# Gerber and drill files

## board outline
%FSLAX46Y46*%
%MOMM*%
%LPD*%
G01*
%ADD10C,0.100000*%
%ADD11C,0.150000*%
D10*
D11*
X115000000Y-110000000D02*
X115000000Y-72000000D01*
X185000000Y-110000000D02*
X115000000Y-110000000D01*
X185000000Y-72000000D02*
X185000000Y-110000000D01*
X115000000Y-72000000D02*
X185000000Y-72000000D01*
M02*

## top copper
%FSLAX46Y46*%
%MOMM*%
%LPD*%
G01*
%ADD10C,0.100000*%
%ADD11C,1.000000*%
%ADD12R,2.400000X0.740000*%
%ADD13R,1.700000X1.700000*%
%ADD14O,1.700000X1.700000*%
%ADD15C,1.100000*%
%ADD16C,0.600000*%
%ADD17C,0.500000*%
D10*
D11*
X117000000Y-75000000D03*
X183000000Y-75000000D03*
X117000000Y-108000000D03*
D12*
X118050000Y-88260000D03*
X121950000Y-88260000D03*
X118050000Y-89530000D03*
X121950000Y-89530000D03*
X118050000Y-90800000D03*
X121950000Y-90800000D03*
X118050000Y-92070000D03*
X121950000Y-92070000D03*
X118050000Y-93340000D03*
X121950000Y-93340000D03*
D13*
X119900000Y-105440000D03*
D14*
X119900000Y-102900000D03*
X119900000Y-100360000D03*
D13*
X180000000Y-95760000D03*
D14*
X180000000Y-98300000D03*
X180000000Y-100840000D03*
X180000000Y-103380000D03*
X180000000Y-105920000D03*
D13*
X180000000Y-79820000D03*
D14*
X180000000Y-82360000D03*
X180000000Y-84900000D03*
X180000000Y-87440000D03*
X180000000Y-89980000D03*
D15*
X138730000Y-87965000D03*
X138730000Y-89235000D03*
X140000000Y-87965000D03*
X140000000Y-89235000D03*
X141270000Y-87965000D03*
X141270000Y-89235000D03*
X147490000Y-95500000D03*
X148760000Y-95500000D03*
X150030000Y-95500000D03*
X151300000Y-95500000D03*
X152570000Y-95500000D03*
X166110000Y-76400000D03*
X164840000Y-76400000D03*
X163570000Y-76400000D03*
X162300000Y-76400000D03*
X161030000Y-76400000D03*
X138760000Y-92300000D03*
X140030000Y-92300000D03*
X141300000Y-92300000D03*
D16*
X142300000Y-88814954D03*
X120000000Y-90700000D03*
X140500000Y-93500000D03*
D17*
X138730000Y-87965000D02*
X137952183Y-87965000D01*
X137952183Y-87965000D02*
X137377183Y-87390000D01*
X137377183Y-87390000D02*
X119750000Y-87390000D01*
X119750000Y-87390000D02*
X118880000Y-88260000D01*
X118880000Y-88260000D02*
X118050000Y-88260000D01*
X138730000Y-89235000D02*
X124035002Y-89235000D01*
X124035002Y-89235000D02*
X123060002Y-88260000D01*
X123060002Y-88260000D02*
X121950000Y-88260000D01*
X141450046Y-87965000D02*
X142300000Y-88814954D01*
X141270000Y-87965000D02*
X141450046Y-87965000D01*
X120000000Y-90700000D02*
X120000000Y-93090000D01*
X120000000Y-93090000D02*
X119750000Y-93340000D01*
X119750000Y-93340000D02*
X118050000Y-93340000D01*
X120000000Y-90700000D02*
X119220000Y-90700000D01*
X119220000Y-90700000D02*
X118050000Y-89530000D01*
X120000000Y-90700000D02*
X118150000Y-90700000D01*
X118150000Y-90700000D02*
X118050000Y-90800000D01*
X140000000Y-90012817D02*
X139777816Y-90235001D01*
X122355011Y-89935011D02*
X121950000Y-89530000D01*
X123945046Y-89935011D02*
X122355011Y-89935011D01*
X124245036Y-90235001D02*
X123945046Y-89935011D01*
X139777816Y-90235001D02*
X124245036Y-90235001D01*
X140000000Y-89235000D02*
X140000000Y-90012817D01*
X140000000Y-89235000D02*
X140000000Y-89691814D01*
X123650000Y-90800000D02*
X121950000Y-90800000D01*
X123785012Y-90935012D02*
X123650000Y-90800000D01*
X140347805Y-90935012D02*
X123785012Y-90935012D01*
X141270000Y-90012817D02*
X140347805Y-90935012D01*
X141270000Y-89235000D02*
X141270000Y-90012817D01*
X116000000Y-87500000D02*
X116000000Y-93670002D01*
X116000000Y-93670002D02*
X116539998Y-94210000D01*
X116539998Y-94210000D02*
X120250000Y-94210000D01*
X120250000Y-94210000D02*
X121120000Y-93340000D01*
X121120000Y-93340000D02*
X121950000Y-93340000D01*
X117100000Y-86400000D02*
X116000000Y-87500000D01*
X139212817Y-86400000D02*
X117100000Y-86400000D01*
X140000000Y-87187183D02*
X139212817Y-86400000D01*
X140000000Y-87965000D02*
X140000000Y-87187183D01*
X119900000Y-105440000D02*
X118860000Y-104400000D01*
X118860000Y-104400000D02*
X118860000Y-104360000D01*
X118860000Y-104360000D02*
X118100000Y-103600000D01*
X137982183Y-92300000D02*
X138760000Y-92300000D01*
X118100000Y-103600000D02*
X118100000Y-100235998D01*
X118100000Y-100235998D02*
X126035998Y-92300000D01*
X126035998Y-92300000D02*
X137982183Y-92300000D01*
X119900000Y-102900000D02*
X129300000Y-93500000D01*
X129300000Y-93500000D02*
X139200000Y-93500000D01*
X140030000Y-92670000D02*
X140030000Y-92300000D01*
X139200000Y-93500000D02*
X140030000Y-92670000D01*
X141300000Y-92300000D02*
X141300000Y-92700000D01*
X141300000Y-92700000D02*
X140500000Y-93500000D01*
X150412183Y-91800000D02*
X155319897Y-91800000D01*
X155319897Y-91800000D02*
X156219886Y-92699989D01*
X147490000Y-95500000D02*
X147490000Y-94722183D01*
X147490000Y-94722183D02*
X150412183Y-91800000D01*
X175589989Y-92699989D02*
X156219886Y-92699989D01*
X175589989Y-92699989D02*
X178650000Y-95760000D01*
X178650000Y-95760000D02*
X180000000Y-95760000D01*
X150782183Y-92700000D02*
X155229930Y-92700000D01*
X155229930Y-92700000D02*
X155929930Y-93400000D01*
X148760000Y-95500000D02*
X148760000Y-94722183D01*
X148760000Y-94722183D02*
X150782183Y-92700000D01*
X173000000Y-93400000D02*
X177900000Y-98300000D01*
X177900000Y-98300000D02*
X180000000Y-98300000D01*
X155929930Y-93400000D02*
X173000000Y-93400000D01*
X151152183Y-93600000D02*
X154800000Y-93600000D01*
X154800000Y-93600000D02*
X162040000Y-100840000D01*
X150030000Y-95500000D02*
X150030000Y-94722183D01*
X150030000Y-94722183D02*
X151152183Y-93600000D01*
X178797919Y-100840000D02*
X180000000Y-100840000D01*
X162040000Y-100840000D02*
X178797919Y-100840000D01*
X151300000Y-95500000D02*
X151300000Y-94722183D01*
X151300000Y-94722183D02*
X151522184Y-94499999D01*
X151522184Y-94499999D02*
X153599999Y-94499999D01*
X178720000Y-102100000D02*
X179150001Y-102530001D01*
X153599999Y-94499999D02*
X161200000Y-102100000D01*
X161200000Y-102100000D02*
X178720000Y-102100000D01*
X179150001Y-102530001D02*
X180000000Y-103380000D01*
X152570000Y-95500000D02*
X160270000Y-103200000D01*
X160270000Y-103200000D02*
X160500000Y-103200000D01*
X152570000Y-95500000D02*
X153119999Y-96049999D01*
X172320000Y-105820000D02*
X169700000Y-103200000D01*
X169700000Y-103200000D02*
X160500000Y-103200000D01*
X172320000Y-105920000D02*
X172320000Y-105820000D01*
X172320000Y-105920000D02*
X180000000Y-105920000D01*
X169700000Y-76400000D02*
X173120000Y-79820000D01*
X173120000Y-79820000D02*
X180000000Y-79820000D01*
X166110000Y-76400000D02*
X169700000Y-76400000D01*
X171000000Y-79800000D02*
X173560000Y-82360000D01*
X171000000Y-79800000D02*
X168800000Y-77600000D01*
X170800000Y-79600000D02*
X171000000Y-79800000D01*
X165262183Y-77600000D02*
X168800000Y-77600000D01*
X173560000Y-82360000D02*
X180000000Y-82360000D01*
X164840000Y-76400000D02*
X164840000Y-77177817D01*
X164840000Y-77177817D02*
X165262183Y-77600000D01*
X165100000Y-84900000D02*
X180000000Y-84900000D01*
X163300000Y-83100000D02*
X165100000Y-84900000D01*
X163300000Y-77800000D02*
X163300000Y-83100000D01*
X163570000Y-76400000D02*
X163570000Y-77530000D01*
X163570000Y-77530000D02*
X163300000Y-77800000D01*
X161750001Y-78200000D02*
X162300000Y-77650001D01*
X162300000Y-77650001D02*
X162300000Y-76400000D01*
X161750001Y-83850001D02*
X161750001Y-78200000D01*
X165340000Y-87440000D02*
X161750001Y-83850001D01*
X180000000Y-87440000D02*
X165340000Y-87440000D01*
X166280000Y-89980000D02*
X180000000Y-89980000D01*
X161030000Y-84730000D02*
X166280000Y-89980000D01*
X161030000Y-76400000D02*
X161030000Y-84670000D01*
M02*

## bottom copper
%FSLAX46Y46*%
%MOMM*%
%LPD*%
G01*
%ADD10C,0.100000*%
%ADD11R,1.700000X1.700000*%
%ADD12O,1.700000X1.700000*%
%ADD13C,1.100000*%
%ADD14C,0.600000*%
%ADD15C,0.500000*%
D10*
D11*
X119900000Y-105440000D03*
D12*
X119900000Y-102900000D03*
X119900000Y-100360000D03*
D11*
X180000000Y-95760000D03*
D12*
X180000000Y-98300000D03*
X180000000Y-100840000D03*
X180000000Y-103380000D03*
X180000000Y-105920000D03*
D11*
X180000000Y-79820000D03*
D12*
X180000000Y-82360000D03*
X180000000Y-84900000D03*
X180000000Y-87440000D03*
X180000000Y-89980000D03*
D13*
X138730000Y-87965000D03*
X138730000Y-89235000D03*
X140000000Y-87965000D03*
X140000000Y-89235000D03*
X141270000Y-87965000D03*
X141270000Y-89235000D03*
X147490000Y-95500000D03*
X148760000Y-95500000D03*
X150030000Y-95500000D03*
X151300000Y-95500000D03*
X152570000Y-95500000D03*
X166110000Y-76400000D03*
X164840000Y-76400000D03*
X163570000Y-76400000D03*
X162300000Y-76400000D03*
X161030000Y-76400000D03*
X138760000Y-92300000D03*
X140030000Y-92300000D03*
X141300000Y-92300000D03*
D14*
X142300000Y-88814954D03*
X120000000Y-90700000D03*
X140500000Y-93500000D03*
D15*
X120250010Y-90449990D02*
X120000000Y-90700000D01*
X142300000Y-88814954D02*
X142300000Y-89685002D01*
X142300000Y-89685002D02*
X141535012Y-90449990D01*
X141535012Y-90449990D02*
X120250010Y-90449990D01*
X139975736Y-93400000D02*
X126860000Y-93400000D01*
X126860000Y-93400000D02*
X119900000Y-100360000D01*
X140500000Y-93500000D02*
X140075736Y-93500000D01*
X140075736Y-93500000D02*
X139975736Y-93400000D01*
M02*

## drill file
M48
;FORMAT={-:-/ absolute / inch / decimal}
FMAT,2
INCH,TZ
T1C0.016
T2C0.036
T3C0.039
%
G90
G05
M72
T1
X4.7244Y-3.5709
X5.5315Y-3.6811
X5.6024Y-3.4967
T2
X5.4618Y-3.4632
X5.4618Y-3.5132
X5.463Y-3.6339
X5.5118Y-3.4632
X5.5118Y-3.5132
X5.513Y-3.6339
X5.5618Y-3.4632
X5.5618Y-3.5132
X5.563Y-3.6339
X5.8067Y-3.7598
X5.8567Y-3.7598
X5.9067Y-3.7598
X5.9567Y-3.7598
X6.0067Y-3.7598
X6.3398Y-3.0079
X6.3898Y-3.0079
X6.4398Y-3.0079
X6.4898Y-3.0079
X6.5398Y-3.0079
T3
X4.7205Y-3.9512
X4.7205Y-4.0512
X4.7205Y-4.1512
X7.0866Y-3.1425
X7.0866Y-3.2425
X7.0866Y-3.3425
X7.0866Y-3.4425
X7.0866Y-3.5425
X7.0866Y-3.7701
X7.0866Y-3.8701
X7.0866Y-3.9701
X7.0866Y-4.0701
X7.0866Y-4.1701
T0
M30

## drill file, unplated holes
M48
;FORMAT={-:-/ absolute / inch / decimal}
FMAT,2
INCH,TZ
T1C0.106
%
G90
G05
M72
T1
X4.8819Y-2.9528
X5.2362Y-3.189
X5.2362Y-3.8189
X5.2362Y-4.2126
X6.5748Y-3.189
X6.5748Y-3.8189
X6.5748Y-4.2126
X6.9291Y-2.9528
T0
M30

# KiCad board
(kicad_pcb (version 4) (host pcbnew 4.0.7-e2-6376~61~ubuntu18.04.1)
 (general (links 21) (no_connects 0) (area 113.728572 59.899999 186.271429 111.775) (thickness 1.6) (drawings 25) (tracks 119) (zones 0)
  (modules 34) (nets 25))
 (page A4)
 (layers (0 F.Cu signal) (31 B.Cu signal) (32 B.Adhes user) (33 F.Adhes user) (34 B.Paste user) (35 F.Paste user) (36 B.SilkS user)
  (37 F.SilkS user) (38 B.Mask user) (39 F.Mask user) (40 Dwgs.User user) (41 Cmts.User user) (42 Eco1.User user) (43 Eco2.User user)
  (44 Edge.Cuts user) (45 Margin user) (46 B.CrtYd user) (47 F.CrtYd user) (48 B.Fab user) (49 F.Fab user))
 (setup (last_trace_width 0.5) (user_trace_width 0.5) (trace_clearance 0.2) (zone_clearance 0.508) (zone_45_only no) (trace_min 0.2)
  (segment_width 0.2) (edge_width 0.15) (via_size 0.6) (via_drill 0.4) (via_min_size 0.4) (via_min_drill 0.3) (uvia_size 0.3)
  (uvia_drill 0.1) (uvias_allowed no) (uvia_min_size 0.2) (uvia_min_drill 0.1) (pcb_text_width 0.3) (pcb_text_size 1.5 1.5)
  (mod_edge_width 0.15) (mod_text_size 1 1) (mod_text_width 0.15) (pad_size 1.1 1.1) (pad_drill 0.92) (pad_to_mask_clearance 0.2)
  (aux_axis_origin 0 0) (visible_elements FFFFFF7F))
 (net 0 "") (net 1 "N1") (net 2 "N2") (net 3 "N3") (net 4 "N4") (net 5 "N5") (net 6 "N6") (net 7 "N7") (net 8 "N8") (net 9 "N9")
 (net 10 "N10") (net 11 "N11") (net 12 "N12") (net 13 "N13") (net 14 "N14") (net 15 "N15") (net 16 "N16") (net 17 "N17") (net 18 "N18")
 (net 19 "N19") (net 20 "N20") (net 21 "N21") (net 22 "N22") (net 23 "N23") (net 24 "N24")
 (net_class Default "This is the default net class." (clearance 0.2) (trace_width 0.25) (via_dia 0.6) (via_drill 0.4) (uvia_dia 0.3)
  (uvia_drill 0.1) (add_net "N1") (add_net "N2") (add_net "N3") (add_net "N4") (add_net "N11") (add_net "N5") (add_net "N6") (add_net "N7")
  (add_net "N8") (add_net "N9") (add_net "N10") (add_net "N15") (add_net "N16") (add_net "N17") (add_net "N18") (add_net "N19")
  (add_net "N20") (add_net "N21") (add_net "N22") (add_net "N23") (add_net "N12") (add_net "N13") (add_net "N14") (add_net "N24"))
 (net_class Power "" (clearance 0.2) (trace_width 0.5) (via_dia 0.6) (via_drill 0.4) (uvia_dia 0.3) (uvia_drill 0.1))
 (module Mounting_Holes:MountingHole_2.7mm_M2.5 (layer F.Cu) (at 176 75)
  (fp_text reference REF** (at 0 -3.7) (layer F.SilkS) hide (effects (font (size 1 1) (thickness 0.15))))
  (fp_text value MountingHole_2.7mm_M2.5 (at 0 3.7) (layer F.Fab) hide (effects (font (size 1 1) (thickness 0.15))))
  (pad 1 np_thru_hole circle (at 0 0) (size 2.7 2.7) (drill 2.7) (layers *.Cu *.Mask)))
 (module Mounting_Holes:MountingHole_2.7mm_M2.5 (layer F.Cu) (at 124 75)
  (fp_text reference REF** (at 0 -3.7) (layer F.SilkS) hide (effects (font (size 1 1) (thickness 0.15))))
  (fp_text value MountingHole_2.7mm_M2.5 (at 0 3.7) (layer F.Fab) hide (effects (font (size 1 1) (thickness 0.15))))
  (pad 1 np_thru_hole circle (at 0 0) (size 2.7 2.7) (drill 2.7) (layers *.Cu *.Mask)))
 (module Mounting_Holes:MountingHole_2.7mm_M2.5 (layer F.Cu) (at 167 107)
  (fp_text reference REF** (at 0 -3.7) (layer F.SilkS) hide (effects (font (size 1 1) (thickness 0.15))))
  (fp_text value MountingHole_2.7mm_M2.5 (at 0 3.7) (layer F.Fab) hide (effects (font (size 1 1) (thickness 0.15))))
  (pad 1 np_thru_hole circle (at 0 0) (size 2.7 2.7) (drill 2.7) (layers *.Cu *.Mask)))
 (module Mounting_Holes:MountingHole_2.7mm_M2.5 (layer F.Cu) (at 133 107)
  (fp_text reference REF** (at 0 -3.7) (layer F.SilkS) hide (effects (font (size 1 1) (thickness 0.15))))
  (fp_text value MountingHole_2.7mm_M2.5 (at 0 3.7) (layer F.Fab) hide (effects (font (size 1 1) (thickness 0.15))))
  (pad 1 np_thru_hole circle (at 0 0) (size 2.7 2.7) (drill 2.7) (layers *.Cu *.Mask)))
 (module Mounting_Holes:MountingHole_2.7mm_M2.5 (layer F.Cu) (at 167 81)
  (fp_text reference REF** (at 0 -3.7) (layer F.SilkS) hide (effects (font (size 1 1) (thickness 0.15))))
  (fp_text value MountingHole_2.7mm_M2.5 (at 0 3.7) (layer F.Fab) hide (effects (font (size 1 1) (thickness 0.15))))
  (pad 1 np_thru_hole circle (at 0 0) (size 2.7 2.7) (drill 2.7) (layers *.Cu *.Mask)))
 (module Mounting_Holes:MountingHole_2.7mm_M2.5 (layer F.Cu) (at 133 97)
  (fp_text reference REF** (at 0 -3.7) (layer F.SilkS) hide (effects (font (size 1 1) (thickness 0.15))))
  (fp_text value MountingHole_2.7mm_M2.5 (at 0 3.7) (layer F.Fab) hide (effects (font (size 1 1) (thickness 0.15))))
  (pad 1 np_thru_hole circle (at 0 0) (size 2.7 2.7) (drill 2.7) (layers *.Cu *.Mask)))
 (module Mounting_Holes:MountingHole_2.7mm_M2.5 (layer F.Cu) (at 167 97)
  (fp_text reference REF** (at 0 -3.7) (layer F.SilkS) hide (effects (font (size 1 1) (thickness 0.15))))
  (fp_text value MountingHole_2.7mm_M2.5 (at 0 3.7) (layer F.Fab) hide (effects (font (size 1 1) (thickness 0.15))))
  (pad 1 np_thru_hole circle (at 0 0) (size 2.7 2.7) (drill 2.7) (layers *.Cu *.Mask)))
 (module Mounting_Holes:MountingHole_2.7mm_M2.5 (layer F.Cu) (at 133 81)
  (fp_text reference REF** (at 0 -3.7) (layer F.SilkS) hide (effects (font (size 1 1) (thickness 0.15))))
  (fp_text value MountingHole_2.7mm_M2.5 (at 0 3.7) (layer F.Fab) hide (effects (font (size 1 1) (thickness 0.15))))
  (pad 1 np_thru_hole circle (at 0 0) (size 2.7 2.7) (drill 2.7) (layers *.Cu *.Mask)))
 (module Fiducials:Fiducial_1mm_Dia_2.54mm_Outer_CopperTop (layer F.Cu) (at 117 75)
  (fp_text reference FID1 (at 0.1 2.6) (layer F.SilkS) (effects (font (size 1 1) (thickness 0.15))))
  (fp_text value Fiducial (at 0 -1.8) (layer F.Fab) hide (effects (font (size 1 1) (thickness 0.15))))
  (pad ~ smd circle (at 0 0) (size 1 1) (layers F.Cu F.Mask) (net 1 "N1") (solder_mask_margin 0.77) (clearance 0.77)))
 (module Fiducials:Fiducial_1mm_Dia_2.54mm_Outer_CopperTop (layer F.Cu) (at 183 75)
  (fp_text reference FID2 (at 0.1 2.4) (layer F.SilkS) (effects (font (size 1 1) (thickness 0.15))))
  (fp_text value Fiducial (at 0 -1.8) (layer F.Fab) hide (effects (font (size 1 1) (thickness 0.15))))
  (pad ~ smd circle (at 0 0) (size 1 1) (layers F.Cu F.Mask) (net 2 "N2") (solder_mask_margin 0.77) (clearance 0.77)))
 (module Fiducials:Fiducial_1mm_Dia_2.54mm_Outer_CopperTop (layer F.Cu) (at 117 108)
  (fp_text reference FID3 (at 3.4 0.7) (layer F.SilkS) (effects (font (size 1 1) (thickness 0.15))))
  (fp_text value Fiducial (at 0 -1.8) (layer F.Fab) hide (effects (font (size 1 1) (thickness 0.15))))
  (pad ~ smd circle (at 0 0) (size 1 1) (layers F.Cu F.Mask) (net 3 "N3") (solder_mask_margin 0.77) (clearance 0.77)))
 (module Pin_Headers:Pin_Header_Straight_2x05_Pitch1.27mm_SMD (layer F.Cu) (at 120 90.8)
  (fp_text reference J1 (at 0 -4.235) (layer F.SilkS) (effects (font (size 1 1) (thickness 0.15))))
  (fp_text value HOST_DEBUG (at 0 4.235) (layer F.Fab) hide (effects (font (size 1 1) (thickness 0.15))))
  (pad 1 smd rect (at -1.95 -2.54) (size 2.4 0.74) (layers F.Cu F.Paste F.Mask) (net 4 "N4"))
  (pad 2 smd rect (at 1.95 -2.54) (size 2.4 0.74) (layers F.Cu F.Paste F.Mask) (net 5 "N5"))
  (pad 3 smd rect (at -1.95 -1.27) (size 2.4 0.74) (layers F.Cu F.Paste F.Mask) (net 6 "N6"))
  (pad 4 smd rect (at 1.95 -1.27) (size 2.4 0.74) (layers F.Cu F.Paste F.Mask) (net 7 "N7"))
  (pad 5 smd rect (at -1.95 0) (size 2.4 0.74) (layers F.Cu F.Paste F.Mask) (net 6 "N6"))
  (pad 6 smd rect (at 1.95 0) (size 2.4 0.74) (layers F.Cu F.Paste F.Mask) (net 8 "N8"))
  (pad 7 smd rect (at -1.95 1.27) (size 2.4 0.74) (layers F.Cu F.Paste F.Mask) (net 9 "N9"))
  (pad 8 smd rect (at 1.95 1.27) (size 2.4 0.74) (layers F.Cu F.Paste F.Mask) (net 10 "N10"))
  (pad 9 smd rect (at -1.95 2.54) (size 2.4 0.74) (layers F.Cu F.Paste F.Mask) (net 6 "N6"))
  (pad 10 smd rect (at 1.95 2.54) (size 2.4 0.74) (layers F.Cu F.Paste F.Mask) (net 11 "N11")))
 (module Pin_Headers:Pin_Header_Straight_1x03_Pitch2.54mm (layer F.Cu) (at 119.9 105.44 180)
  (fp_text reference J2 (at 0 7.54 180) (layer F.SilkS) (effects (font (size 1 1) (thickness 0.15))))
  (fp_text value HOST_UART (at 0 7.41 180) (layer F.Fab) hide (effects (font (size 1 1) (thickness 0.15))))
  (pad 1 thru_hole rect (at 0 0 180) (size 1.7 1.7) (drill 1) (layers *.Cu *.Mask) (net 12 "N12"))
  (pad 2 thru_hole oval (at 0 2.54 180) (size 1.7 1.7) (drill 1) (layers *.Cu *.Mask) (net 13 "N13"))
  (pad 3 thru_hole oval (at 0 5.08 180) (size 1.7 1.7) (drill 1) (layers *.Cu *.Mask) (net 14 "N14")))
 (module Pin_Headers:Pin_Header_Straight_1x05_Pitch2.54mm (layer F.Cu) (at 180 95.76)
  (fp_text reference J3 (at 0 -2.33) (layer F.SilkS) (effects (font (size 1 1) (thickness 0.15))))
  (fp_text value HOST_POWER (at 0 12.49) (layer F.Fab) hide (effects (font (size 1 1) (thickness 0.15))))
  (pad 1 thru_hole rect (at 0 0) (size 1.7 1.7) (drill 1) (layers *.Cu *.Mask) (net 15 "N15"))
  (pad 2 thru_hole oval (at 0 2.54) (size 1.7 1.7) (drill 1) (layers *.Cu *.Mask) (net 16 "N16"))
  (pad 3 thru_hole oval (at 0 5.08) (size 1.7 1.7) (drill 1) (layers *.Cu *.Mask) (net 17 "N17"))
  (pad 4 thru_hole oval (at 0 7.62) (size 1.7 1.7) (drill 1) (layers *.Cu *.Mask) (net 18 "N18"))
  (pad 5 thru_hole oval (at 0 10.16) (size 1.7 1.7) (drill 1) (layers *.Cu *.Mask) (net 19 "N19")))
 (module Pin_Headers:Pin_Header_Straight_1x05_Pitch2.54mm (layer F.Cu) (at 180 79.82)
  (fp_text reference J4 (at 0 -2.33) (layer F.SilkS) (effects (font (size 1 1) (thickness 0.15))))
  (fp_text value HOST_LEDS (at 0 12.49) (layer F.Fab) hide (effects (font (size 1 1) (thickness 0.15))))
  (pad 1 thru_hole rect (at 0 0) (size 1.7 1.7) (drill 1) (layers *.Cu *.Mask) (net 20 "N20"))
  (pad 2 thru_hole oval (at 0 2.54) (size 1.7 1.7) (drill 1) (layers *.Cu *.Mask) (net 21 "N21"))
  (pad 3 thru_hole oval (at 0 5.08) (size 1.7 1.7) (drill 1) (layers *.Cu *.Mask) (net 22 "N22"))
  (pad 4 thru_hole oval (at 0 7.62) (size 1.7 1.7) (drill 1) (layers *.Cu *.Mask) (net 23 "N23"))
  (pad 5 thru_hole oval (at 0 10.16) (size 1.7 1.7) (drill 1) (layers *.Cu *.Mask) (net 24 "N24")))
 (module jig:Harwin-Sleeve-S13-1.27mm (layer F.Cu) (at 138.73 87.965)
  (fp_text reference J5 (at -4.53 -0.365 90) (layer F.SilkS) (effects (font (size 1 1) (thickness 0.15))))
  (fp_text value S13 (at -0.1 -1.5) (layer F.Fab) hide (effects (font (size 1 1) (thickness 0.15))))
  (pad 1 thru_hole circle (at 0 0) (size 1.1 1.1) (drill 0.92) (layers *.Cu *.Mask) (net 4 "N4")))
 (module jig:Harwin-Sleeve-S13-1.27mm (layer F.Cu) (at 138.73 89.235)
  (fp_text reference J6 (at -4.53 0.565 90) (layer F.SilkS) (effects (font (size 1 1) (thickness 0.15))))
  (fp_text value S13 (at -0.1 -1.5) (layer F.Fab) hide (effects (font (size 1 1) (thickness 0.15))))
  (pad 1 thru_hole circle (at 0 0) (size 1.1 1.1) (drill 0.92) (layers *.Cu *.Mask) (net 5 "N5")))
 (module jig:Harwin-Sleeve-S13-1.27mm (layer F.Cu) (at 140 87.965)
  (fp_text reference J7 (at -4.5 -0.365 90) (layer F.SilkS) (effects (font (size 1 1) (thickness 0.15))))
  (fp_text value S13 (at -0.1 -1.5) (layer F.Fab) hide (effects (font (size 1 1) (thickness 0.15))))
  (pad 1 thru_hole circle (at 0 0) (size 1.1 1.1) (drill 0.92) (layers *.Cu *.Mask) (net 11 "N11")))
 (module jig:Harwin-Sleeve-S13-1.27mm (layer F.Cu) (at 140 89.235)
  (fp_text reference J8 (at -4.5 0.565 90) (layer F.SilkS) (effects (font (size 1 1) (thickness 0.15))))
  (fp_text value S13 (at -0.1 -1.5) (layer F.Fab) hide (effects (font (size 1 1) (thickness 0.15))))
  (pad 1 thru_hole circle (at 0 0) (size 1.1 1.1) (drill 0.92) (layers *.Cu *.Mask) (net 7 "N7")))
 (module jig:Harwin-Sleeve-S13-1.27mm (layer F.Cu) (at 141.27 87.965)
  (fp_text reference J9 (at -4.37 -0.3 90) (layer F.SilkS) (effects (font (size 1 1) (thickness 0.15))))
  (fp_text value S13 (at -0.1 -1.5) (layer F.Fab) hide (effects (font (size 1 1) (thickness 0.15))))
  (pad 1 thru_hole circle (at 0 0) (size 1.1 1.1) (drill 0.92) (layers *.Cu *.Mask) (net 6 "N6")))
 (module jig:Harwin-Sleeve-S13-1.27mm (layer F.Cu) (at 141.27 89.235)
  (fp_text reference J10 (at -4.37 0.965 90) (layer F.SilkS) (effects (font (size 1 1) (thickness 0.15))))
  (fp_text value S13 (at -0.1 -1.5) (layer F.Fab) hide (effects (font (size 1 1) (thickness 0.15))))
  (pad 1 thru_hole circle (at 0 0) (size 1.1 1.1) (drill 0.92) (layers *.Cu *.Mask) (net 8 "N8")))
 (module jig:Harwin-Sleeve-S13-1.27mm (layer F.Cu) (at 147.49 93.5)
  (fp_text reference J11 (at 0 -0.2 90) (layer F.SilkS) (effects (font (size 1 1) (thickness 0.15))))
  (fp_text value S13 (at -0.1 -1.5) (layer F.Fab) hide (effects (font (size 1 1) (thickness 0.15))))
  (pad 1 thru_hole circle (at 0 2) (size 1.1 1.1) (drill 0.92) (layers *.Cu *.Mask) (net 15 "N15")))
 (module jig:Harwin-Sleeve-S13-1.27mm (layer F.Cu) (at 148.76 93.5)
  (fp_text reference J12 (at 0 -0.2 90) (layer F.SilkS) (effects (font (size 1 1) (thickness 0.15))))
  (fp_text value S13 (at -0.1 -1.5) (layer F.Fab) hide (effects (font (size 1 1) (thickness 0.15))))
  (pad 1 thru_hole circle (at 0 2) (size 1.1 1.1) (drill 0.92) (layers *.Cu *.Mask) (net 16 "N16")))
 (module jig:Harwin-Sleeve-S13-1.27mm (layer F.Cu) (at 150.03 93.5)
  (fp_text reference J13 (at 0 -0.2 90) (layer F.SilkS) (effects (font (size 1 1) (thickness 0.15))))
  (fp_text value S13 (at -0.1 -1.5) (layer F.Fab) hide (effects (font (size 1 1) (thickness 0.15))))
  (pad 1 thru_hole circle (at 0 2) (size 1.1 1.1) (drill 0.92) (layers *.Cu *.Mask) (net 17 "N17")))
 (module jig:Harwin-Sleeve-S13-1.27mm (layer F.Cu) (at 151.3 93.5)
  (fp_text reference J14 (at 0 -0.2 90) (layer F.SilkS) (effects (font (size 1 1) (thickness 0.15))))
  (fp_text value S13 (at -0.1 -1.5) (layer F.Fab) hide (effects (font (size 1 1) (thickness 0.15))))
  (pad 1 thru_hole circle (at 0 2) (size 1.1 1.1) (drill 0.92) (layers *.Cu *.Mask) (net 18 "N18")))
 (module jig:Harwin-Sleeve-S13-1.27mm (layer F.Cu) (at 152.57 93.5)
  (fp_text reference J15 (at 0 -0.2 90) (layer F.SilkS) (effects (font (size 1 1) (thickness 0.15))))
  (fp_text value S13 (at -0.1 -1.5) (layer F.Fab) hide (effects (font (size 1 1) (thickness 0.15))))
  (pad 1 thru_hole circle (at 0 2) (size 1.1 1.1) (drill 0.92) (layers *.Cu *.Mask) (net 19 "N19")))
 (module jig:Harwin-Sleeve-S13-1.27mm (layer F.Cu) (at 166.11 76.4)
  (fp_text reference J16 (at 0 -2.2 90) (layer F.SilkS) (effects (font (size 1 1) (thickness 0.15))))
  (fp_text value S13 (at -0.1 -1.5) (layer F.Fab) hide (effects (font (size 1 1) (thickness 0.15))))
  (pad 1 thru_hole circle (at 0 0) (size 1.1 1.1) (drill 0.92) (layers *.Cu *.Mask) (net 20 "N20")))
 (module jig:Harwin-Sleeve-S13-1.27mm (layer F.Cu) (at 164.84 76.4)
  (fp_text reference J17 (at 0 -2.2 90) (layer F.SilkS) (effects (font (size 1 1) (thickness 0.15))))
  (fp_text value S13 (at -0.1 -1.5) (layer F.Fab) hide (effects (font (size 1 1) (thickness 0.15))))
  (pad 1 thru_hole circle (at 0 0) (size 1.1 1.1) (drill 0.92) (layers *.Cu *.Mask) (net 21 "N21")))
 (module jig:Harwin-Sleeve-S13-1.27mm (layer F.Cu) (at 163.57 76.4)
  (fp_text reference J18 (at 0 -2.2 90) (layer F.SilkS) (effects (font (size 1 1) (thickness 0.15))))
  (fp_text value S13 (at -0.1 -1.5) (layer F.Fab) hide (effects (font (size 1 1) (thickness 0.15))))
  (pad 1 thru_hole circle (at 0 0) (size 1.1 1.1) (drill 0.92) (layers *.Cu *.Mask) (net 22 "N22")))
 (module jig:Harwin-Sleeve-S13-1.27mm (layer F.Cu) (at 162.3 76.4)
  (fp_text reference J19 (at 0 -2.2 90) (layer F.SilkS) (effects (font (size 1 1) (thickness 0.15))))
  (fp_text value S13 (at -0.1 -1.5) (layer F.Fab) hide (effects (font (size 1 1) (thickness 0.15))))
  (pad 1 thru_hole circle (at 0 0) (size 1.1 1.1) (drill 0.92) (layers *.Cu *.Mask) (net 23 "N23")))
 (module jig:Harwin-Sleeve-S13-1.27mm (layer F.Cu) (at 161.03 76.4)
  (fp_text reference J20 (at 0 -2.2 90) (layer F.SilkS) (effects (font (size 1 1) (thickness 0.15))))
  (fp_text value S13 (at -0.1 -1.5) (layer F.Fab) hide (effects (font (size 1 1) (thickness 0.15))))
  (pad 1 thru_hole circle (at 0 0) (size 1.1 1.1) (drill 0.92) (layers *.Cu *.Mask) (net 24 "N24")))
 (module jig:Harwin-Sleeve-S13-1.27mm (layer F.Cu) (at 138.76 92.3)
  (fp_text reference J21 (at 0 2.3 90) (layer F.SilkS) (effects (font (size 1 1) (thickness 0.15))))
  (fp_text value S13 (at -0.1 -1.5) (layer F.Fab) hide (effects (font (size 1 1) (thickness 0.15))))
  (pad 1 thru_hole circle (at 0 0) (size 1.1 1.1) (drill 0.92) (layers *.Cu *.Mask) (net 12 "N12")))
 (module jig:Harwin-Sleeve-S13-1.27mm (layer F.Cu) (at 140.03 92.3)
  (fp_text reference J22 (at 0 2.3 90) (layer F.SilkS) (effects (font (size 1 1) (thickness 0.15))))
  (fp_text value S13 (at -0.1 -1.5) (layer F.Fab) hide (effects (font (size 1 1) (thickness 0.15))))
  (pad 1 thru_hole circle (at 0 0) (size 1.1 1.1) (drill 0.92) (layers *.Cu *.Mask) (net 13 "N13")))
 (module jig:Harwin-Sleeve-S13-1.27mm (layer F.Cu) (at 141.3 92.3)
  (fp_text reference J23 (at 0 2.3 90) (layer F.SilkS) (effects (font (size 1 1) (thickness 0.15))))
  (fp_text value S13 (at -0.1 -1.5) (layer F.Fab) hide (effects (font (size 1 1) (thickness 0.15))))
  (pad 1 thru_hole circle (at 0 0) (size 1.1 1.1) (drill 0.92) (layers *.Cu *.Mask) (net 14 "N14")))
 (gr_line (start 115 110) (end 115 72) (layer Edge.Cuts) (width 0.15))
 (gr_line (start 185 110) (end 115 110) (layer Edge.Cuts) (width 0.15))
 (gr_line (start 185 72) (end 185 110) (layer Edge.Cuts) (width 0.15))
 (gr_line (start 115 72) (end 185 72) (layer Edge.Cuts) (width 0.15))
 (segment (start 138.73 87.965) (end 137.952183 87.965) (width 0.5) (layer F.Cu) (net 4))
 (segment (start 137.952183 87.965) (end 137.377183 87.39) (width 0.5) (layer F.Cu) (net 4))
 (segment (start 137.377183 87.39) (end 119.75 87.39) (width 0.5) (layer F.Cu) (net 4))
 (segment (start 119.75 87.39) (end 118.88 88.26) (width 0.5) (layer F.Cu) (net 4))
 (segment (start 118.88 88.26) (end 118.05 88.26) (width 0.5) (layer F.Cu) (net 4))
 (segment (start 138.73 89.235) (end 124.035002 89.235) (width 0.5) (layer F.Cu) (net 5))
 (segment (start 124.035002 89.235) (end 123.060002 88.26) (width 0.5) (layer F.Cu) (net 5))
 (segment (start 123.060002 88.26) (end 121.95 88.26) (width 0.5) (layer F.Cu) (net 5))
 (segment (start 120.25001 90.44999) (end 120 90.7) (width 0.5) (layer B.Cu) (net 6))
 (segment (start 142.3 88.814954) (end 142.3 89.685002) (width 0.5) (layer B.Cu) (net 6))
 (segment (start 142.3 89.685002) (end 141.535012 90.44999) (width 0.5) (layer B.Cu) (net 6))
 (segment (start 141.535012 90.44999) (end 120.25001 90.44999) (width 0.5) (layer B.Cu) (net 6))
 (via (at 142.3 88.814954) (size 0.6) (drill 0.4) (layers F.Cu B.Cu) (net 6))
 (segment (start 141.450046 87.965) (end 142.3 88.814954) (width 0.5) (layer F.Cu) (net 6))
 (segment (start 141.27 87.965) (end 141.450046 87.965) (width 0.5) (layer F.Cu) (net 6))
 (segment (start 120 90.7) (end 120 93.09) (width 0.5) (layer F.Cu) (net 6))
 (segment (start 120 93.09) (end 119.75 93.34) (width 0.5) (layer F.Cu) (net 6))
 (segment (start 119.75 93.34) (end 118.05 93.34) (width 0.5) (layer F.Cu) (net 6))
 (segment (start 120 90.7) (end 119.22 90.7) (width 0.5) (layer F.Cu) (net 6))
 (segment (start 119.22 90.7) (end 118.05 89.53) (width 0.5) (layer F.Cu) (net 6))
 (segment (start 120 90.7) (end 118.15 90.7) (width 0.5) (layer F.Cu) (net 6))
 (segment (start 118.15 90.7) (end 118.05 90.8) (width 0.5) (layer F.Cu) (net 6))
 (via (at 120 90.7) (size 0.6) (drill 0.4) (layers F.Cu B.Cu) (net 6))
 (segment (start 140 90.012817) (end 139.777816 90.235001) (width 0.5) (layer F.Cu) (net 7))
 (segment (start 122.355011 89.935011) (end 121.95 89.53) (width 0.5) (layer F.Cu) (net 7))
 (segment (start 123.945046 89.935011) (end 122.355011 89.935011) (width 0.5) (layer F.Cu) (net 7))
 (segment (start 124.245036 90.235001) (end 123.945046 89.935011) (width 0.5) (layer F.Cu) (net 7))
 (segment (start 139.777816 90.235001) (end 124.245036 90.235001) (width 0.5) (layer F.Cu) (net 7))
 (segment (start 140 89.235) (end 140 90.012817) (width 0.5) (layer F.Cu) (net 7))
 (segment (start 140 89.235) (end 140 89.691814) (width 0.5) (layer F.Cu) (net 7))
 (segment (start 123.65 90.8) (end 121.95 90.8) (width 0.5) (layer F.Cu) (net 8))
 (segment (start 123.785012 90.935012) (end 123.65 90.8) (width 0.5) (layer F.Cu) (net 8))
 (segment (start 140.347805 90.935012) (end 123.785012 90.935012) (width 0.5) (layer F.Cu) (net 8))
 (segment (start 141.27 90.012817) (end 140.347805 90.935012) (width 0.5) (layer F.Cu) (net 8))
 (segment (start 141.27 89.235) (end 141.27 90.012817) (width 0.5) (layer F.Cu) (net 8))
 (segment (start 116 87.5) (end 116 93.670002) (width 0.5) (layer F.Cu) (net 11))
 (segment (start 116 93.670002) (end 116.539998 94.21) (width 0.5) (layer F.Cu) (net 11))
 (segment (start 116.539998 94.21) (end 120.25 94.21) (width 0.5) (layer F.Cu) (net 11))
 (segment (start 120.25 94.21) (end 121.12 93.34) (width 0.5) (layer F.Cu) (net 11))
 (segment (start 121.12 93.34) (end 121.95 93.34) (width 0.5) (layer F.Cu) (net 11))
 (segment (start 117.1 86.4) (end 116 87.5) (width 0.5) (layer F.Cu) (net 11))
 (segment (start 139.212817 86.4) (end 117.1 86.4) (width 0.5) (layer F.Cu) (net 11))
 (segment (start 140 87.187183) (end 139.212817 86.4) (width 0.5) (layer F.Cu) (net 11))
 (segment (start 140 87.965) (end 140 87.187183) (width 0.5) (layer F.Cu) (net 11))
 (segment (start 119.9 105.44) (end 118.86 104.4) (width 0.5) (layer F.Cu) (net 12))
 (segment (start 118.86 104.4) (end 118.86 104.36) (width 0.5) (layer F.Cu) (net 12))
 (segment (start 118.86 104.36) (end 118.1 103.6) (width 0.5) (layer F.Cu) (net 12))
 (segment (start 137.982183 92.3) (end 138.76 92.3) (width 0.5) (layer F.Cu) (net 12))
 (segment (start 118.1 103.6) (end 118.1 100.235998) (width 0.5) (layer F.Cu) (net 12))
 (segment (start 118.1 100.235998) (end 126.035998 92.3) (width 0.5) (layer F.Cu) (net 12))
 (segment (start 126.035998 92.3) (end 137.982183 92.3) (width 0.5) (layer F.Cu) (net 12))
 (segment (start 119.9 102.9) (end 129.3 93.5) (width 0.5) (layer F.Cu) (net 13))
 (segment (start 129.3 93.5) (end 139.2 93.5) (width 0.5) (layer F.Cu) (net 13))
 (segment (start 140.03 92.67) (end 140.03 92.3) (width 0.5) (layer F.Cu) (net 13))
 (segment (start 139.2 93.5) (end 140.03 92.67) (width 0.5) (layer F.Cu) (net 13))
 (segment (start 139.975736 93.4) (end 126.86 93.4) (width 0.5) (layer B.Cu) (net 14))
 (segment (start 126.86 93.4) (end 119.9 100.36) (width 0.5) (layer B.Cu) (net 14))
 (segment (start 140.5 93.5) (end 140.075736 93.5) (width 0.5) (layer B.Cu) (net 14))
 (segment (start 140.075736 93.5) (end 139.975736 93.4) (width 0.5) (layer B.Cu) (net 14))
 (segment (start 141.3 92.3) (end 141.3 92.7) (width 0.5) (layer F.Cu) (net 14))
 (segment (start 141.3 92.7) (end 140.5 93.5) (width 0.5) (layer F.Cu) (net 14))
 (via (at 140.5 93.5) (size 0.6) (drill 0.4) (layers F.Cu B.Cu) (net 14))
 (segment (start 150.412183 91.8) (end 155.319897 91.8) (width 0.5) (layer F.Cu) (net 15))
 (segment (start 155.319897 91.8) (end 156.219886 92.699989) (width 0.5) (layer F.Cu) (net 15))
 (segment (start 147.49 95.5) (end 147.49 94.722183) (width 0.5) (layer F.Cu) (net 15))
 (segment (start 147.49 94.722183) (end 150.412183 91.8) (width 0.5) (layer F.Cu) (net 15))
 (segment (start 175.589989 92.699989) (end 156.219886 92.699989) (width 0.5) (layer F.Cu) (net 15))
 (segment (start 175.589989 92.699989) (end 178.65 95.76) (width 0.5) (layer F.Cu) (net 15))
 (segment (start 178.65 95.76) (end 180 95.76) (width 0.5) (layer F.Cu) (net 15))
 (segment (start 150.782183 92.7) (end 155.22993 92.7) (width 0.5) (layer F.Cu) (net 16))
 (segment (start 155.22993 92.7) (end 155.92993 93.4) (width 0.5) (layer F.Cu) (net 16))
 (segment (start 148.76 95.5) (end 148.76 94.722183) (width 0.5) (layer F.Cu) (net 16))
 (segment (start 148.76 94.722183) (end 150.782183 92.7) (width 0.5) (layer F.Cu) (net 16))
 (segment (start 173 93.4) (end 177.9 98.3) (width 0.5) (layer F.Cu) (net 16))
 (segment (start 177.9 98.3) (end 180 98.3) (width 0.5) (layer F.Cu) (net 16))
 (segment (start 155.92993 93.4) (end 173 93.4) (width 0.5) (layer F.Cu) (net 16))
 (segment (start 151.152183 93.6) (end 154.8 93.6) (width 0.5) (layer F.Cu) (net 17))
 (segment (start 154.8 93.6) (end 162.04 100.84) (width 0.5) (layer F.Cu) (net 17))
 (segment (start 150.03 95.5) (end 150.03 94.722183) (width 0.5) (layer F.Cu) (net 17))
 (segment (start 150.03 94.722183) (end 151.152183 93.6) (width 0.5) (layer F.Cu) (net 17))
 (segment (start 178.797919 100.84) (end 180 100.84) (width 0.5) (layer F.Cu) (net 17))
 (segment (start 162.04 100.84) (end 178.797919 100.84) (width 0.5) (layer F.Cu) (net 17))
 (segment (start 151.3 95.5) (end 151.3 94.722183) (width 0.5) (layer F.Cu) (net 18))
 (segment (start 151.3 94.722183) (end 151.522184 94.499999) (width 0.5) (layer F.Cu) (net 18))
 (segment (start 151.522184 94.499999) (end 153.599999 94.499999) (width 0.5) (layer F.Cu) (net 18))
 (segment (start 178.72 102.1) (end 179.150001 102.530001) (width 0.5) (layer F.Cu) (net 18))
 (segment (start 153.599999 94.499999) (end 161.2 102.1) (width 0.5) (layer F.Cu) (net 18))
 (segment (start 161.2 102.1) (end 178.72 102.1) (width 0.5) (layer F.Cu) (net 18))
 (segment (start 179.150001 102.530001) (end 180 103.38) (width 0.5) (layer F.Cu) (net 18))
 (segment (start 152.57 95.5) (end 160.27 103.2) (width 0.5) (layer F.Cu) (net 19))
 (segment (start 160.27 103.2) (end 160.5 103.2) (width 0.5) (layer F.Cu) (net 19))
 (segment (start 152.57 95.5) (end 153.119999 96.049999) (width 0.5) (layer F.Cu) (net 19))
 (segment (start 172.32 105.82) (end 169.7 103.2) (width 0.5) (layer F.Cu) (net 19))
 (segment (start 169.7 103.2) (end 160.5 103.2) (width 0.5) (layer F.Cu) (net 19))
 (segment (start 172.32 105.92) (end 172.32 105.82) (width 0.5) (layer F.Cu) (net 19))
 (segment (start 172.32 105.92) (end 180 105.92) (width 0.5) (layer F.Cu) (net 19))
 (segment (start 169.7 76.4) (end 173.12 79.82) (width 0.5) (layer F.Cu) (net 20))
 (segment (start 173.12 79.82) (end 180 79.82) (width 0.5) (layer F.Cu) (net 20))
 (segment (start 166.11 76.4) (end 169.7 76.4) (width 0.5) (layer F.Cu) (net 20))
 (segment (start 171 79.8) (end 173.56 82.36) (width 0.5) (layer F.Cu) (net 21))
 (segment (start 171 79.8) (end 168.8 77.6) (width 0.5) (layer F.Cu) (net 21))
 (segment (start 170.8 79.6) (end 171 79.8) (width 0.5) (layer F.Cu) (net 21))
 (segment (start 165.262183 77.6) (end 168.8 77.6) (width 0.5) (layer F.Cu) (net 21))
 (segment (start 173.56 82.36) (end 180 82.36) (width 0.5) (layer F.Cu) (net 21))
 (segment (start 164.84 76.4) (end 164.84 77.177817) (width 0.5) (layer F.Cu) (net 21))
 (segment (start 164.84 77.177817) (end 165.262183 77.6) (width 0.5) (layer F.Cu) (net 21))
 (segment (start 165.1 84.9) (end 180 84.9) (width 0.5) (layer F.Cu) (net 22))
 (segment (start 163.3 83.1) (end 165.1 84.9) (width 0.5) (layer F.Cu) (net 22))
 (segment (start 163.3 77.8) (end 163.3 83.1) (width 0.5) (layer F.Cu) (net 22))
 (segment (start 163.57 76.4) (end 163.57 77.53) (width 0.5) (layer F.Cu) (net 22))
 (segment (start 163.57 77.53) (end 163.3 77.8) (width 0.5) (layer F.Cu) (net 22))
 (segment (start 161.750001 78.2) (end 162.3 77.650001) (width 0.5) (layer F.Cu) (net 23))
 (segment (start 162.3 77.650001) (end 162.3 76.4) (width 0.5) (layer F.Cu) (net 23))
 (segment (start 161.750001 83.850001) (end 161.750001 78.2) (width 0.5) (layer F.Cu) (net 23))
 (segment (start 165.34 87.44) (end 161.750001 83.850001) (width 0.5) (layer F.Cu) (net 23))
 (segment (start 180 87.44) (end 165.34 87.44) (width 0.5) (layer F.Cu) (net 23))
 (segment (start 166.28 89.98) (end 180 89.98) (width 0.5) (layer F.Cu) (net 24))
 (segment (start 161.03 84.73) (end 166.28 89.98) (width 0.5) (layer F.Cu) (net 24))
 (segment (start 161.03 76.4) (end 161.03 84.67) (width 0.5) (layer F.Cu) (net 24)))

